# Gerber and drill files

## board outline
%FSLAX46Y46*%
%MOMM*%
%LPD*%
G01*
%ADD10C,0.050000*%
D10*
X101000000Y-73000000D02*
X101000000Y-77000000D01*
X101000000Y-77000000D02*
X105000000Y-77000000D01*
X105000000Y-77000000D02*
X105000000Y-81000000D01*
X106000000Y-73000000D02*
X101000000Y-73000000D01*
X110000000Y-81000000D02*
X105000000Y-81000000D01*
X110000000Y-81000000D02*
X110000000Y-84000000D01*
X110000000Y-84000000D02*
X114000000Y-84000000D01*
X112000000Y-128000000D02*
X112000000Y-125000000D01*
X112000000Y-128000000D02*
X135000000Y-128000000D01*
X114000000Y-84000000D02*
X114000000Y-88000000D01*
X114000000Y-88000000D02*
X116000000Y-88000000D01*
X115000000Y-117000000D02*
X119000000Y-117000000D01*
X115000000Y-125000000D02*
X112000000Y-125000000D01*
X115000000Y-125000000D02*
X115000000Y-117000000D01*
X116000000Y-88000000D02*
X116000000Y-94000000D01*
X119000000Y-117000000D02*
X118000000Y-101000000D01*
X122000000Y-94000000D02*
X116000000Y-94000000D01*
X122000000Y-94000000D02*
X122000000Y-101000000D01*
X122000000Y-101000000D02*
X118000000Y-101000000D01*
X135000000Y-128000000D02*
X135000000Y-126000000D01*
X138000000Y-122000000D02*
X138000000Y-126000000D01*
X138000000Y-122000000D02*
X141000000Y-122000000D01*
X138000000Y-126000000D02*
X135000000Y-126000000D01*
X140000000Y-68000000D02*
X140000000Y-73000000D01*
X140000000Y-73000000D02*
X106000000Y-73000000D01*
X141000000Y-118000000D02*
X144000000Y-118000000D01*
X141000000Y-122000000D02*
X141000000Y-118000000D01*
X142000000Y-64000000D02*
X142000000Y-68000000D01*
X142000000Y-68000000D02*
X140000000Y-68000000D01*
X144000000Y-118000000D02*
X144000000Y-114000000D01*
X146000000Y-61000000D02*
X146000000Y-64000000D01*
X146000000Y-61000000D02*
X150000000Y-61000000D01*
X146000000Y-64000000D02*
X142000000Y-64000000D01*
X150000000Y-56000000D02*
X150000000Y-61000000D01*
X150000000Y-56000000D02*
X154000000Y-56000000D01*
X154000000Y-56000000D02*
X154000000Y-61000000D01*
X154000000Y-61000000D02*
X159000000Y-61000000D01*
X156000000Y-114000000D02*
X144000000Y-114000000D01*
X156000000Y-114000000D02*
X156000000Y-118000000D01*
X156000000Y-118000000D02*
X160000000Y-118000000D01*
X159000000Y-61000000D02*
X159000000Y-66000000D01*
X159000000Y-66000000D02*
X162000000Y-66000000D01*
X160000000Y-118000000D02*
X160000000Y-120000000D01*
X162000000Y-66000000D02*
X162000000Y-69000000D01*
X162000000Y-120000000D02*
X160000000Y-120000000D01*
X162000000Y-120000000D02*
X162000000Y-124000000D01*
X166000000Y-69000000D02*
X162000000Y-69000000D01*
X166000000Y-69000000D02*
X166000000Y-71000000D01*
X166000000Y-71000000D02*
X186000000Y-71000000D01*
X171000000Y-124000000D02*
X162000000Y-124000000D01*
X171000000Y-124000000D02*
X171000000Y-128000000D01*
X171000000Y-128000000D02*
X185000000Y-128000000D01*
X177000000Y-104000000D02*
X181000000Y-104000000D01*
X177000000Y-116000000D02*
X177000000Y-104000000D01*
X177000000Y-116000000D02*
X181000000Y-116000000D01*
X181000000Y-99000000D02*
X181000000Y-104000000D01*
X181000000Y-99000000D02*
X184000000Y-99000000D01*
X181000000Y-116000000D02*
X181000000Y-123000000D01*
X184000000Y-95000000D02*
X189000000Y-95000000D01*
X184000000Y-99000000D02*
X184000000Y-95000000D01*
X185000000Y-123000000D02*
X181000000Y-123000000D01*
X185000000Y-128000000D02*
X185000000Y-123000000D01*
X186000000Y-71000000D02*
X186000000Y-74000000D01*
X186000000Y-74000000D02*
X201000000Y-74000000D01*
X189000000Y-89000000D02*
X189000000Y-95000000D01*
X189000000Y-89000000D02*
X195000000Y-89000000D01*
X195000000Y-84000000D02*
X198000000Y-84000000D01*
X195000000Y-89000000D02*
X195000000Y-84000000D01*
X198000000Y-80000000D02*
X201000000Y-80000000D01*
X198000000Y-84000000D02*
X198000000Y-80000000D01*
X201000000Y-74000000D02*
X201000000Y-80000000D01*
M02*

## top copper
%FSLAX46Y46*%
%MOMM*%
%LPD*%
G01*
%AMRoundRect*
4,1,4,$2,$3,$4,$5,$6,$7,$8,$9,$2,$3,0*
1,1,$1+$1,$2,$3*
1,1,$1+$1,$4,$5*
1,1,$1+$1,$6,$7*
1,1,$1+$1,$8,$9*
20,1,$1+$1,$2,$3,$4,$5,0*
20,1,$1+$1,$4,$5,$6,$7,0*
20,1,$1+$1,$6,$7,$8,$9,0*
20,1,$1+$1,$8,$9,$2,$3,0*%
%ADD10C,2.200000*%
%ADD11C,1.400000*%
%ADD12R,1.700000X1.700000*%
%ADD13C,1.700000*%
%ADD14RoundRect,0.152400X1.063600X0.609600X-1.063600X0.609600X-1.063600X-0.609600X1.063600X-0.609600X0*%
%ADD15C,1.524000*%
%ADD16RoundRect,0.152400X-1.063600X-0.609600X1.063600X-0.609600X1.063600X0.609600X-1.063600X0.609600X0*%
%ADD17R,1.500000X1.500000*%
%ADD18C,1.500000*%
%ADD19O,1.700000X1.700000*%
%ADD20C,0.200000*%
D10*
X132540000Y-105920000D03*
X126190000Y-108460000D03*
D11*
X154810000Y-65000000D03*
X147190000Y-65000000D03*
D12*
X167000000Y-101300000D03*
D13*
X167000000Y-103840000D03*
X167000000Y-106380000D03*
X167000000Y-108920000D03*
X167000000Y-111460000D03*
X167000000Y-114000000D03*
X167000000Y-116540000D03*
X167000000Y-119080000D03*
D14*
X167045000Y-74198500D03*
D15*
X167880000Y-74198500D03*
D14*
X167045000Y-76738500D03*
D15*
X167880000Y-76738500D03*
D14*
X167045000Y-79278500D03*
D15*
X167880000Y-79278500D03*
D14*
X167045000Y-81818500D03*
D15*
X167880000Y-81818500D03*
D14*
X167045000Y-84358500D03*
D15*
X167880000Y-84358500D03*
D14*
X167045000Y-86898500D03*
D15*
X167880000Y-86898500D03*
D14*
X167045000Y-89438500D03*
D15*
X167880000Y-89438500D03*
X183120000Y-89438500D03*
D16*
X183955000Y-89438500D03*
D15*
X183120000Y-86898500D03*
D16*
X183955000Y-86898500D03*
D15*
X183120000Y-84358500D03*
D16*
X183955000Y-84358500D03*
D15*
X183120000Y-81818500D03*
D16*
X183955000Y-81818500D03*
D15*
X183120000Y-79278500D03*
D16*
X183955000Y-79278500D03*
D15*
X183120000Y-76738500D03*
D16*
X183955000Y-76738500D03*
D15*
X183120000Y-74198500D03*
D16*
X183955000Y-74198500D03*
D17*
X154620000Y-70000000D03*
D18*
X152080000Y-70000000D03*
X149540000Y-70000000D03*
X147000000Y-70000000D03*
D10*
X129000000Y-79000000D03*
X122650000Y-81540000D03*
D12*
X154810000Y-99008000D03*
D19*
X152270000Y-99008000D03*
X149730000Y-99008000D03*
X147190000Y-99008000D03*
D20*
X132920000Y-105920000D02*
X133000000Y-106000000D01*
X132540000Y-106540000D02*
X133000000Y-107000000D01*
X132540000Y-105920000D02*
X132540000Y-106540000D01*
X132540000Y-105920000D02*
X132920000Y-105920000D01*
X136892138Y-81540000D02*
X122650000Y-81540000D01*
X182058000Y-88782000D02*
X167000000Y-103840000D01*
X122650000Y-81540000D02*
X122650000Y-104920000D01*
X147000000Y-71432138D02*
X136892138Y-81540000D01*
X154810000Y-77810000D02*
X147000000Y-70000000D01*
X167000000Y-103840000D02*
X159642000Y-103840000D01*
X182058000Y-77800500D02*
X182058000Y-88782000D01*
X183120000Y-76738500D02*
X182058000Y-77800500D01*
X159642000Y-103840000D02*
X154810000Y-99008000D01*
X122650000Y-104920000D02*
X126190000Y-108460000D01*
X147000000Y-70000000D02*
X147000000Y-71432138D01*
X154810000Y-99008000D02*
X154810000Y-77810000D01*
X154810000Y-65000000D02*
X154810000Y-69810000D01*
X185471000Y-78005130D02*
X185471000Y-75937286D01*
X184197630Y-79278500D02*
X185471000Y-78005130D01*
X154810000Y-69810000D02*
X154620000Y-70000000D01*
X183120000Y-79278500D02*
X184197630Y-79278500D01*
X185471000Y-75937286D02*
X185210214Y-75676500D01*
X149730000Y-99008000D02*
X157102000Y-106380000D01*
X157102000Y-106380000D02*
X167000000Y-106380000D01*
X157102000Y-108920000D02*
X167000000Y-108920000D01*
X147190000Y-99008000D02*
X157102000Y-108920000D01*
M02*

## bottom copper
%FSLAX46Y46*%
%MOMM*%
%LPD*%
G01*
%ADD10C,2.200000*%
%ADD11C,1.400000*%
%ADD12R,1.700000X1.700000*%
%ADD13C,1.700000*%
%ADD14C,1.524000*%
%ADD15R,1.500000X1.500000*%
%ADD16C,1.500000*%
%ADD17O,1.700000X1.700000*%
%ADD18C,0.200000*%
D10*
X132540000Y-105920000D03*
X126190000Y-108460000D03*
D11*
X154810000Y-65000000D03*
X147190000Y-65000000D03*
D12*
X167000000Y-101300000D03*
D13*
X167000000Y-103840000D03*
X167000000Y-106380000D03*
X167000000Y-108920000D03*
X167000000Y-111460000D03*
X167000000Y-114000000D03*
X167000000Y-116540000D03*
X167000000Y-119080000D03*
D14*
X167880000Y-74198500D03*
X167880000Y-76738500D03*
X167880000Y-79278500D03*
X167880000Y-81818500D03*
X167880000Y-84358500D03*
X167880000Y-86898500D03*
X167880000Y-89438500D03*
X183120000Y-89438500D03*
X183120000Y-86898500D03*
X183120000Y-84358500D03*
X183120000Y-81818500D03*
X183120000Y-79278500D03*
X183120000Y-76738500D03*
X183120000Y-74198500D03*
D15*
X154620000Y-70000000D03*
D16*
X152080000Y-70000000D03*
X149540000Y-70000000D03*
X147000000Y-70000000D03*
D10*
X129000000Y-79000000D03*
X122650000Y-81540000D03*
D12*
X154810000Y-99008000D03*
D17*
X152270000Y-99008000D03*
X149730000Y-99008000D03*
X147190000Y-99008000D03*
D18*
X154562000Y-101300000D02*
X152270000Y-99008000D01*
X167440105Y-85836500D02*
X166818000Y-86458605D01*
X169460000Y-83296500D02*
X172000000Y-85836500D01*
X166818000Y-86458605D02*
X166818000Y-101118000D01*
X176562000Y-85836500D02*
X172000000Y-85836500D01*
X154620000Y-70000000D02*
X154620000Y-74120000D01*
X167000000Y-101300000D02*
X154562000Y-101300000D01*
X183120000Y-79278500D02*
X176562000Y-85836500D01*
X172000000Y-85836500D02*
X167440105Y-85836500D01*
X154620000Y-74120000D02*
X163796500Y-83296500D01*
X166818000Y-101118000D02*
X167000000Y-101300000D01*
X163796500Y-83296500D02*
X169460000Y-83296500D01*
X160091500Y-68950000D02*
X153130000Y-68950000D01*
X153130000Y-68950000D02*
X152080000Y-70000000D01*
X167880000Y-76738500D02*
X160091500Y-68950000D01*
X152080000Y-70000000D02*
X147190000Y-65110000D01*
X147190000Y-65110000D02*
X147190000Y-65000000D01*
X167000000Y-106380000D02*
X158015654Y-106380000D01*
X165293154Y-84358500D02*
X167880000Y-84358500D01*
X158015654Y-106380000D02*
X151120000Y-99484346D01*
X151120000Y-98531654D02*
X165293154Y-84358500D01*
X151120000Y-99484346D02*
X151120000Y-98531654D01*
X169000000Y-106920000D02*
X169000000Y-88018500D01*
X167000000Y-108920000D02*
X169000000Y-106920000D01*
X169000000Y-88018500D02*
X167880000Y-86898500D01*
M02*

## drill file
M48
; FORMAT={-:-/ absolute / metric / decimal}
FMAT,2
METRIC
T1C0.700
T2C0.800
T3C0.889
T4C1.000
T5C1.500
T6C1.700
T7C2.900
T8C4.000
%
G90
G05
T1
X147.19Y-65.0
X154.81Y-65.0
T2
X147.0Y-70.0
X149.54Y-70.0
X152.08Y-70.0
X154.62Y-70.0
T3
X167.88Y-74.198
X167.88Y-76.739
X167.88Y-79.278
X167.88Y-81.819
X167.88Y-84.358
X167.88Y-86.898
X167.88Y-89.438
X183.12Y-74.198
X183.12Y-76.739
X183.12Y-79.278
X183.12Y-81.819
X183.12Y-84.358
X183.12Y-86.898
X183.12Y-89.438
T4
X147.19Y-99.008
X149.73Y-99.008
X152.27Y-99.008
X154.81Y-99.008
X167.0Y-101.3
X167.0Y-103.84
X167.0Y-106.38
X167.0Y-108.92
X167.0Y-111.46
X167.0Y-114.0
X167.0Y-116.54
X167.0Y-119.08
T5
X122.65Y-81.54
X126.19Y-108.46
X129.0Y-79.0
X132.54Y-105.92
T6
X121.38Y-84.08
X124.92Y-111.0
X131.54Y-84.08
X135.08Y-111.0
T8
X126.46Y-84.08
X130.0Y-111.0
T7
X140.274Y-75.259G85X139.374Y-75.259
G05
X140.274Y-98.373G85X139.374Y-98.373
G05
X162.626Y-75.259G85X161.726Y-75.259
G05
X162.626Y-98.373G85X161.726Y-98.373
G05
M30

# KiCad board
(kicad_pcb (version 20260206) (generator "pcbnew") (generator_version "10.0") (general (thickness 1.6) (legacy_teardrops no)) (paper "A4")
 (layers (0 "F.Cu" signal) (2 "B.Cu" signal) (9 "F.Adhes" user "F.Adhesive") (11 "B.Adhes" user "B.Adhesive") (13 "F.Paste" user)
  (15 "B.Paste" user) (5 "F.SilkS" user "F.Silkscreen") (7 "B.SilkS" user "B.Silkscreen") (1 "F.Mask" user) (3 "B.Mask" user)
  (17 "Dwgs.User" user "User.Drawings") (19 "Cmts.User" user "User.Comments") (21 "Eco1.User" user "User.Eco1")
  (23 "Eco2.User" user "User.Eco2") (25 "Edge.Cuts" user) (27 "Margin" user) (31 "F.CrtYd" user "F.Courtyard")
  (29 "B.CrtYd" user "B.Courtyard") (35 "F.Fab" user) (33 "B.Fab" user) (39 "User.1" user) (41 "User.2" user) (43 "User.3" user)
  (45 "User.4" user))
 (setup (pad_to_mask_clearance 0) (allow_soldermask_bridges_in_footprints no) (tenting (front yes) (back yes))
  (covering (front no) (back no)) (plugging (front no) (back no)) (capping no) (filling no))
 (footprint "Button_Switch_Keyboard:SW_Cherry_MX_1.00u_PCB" (layer "F.Cu") (at 132.54 105.92)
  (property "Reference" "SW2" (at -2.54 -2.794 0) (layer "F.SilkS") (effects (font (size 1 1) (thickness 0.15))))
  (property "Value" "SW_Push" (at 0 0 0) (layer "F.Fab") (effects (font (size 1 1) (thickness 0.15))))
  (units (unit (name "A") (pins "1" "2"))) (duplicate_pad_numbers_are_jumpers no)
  (pad "" np_thru_hole circle (at -7.62 5.08) (size 1.7 1.7) (drill 1.7) (layers "*.Cu" "*.Mask"))
  (pad "" np_thru_hole circle (at -2.54 5.08) (size 4 4) (drill 4) (layers "*.Cu" "*.Mask"))
  (pad "" np_thru_hole circle (at 2.54 5.08) (size 1.7 1.7) (drill 1.7) (layers "*.Cu" "*.Mask"))
  (pad "1" thru_hole circle (at 0 0) (size 2.2 2.2) (drill 1.5) (layers "*.Cu" "*.Mask") (remove_unused_layers no) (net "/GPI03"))
  (pad "2" thru_hole circle (at -6.35 2.54) (size 2.2 2.2) (drill 1.5) (layers "*.Cu" "*.Mask") (remove_unused_layers no) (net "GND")))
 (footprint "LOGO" (layer "F.Cu") (at 160 112)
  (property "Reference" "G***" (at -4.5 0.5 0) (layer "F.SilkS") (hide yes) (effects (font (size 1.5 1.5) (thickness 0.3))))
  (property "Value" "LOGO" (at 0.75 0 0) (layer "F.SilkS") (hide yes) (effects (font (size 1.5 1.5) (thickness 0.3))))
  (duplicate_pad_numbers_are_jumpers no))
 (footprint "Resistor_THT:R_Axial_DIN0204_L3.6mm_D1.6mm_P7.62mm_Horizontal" (layer "F.Cu") (at 154.81 65 180)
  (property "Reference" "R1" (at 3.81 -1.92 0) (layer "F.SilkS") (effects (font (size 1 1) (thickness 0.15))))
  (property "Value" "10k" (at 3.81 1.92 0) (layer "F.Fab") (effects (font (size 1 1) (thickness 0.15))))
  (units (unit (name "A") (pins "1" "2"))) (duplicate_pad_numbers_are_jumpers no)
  (pad "1" thru_hole circle (at 0 0 180) (size 1.4 1.4) (drill 0.7) (layers "*.Cu" "*.Mask") (remove_unused_layers no) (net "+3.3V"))
  (pad "2" thru_hole circle (at 7.62 0 180) (size 1.4 1.4) (drill 0.7) (layers "*.Cu" "*.Mask") (remove_unused_layers no)
   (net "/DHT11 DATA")))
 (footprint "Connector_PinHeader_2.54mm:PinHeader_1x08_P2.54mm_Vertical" (layer "F.Cu") (at 167 101.3)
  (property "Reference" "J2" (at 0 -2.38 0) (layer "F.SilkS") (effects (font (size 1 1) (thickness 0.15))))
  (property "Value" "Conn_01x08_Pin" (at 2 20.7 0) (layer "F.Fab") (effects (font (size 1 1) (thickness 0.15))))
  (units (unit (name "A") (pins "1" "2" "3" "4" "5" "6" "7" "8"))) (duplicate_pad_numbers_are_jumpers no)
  (pad "1" thru_hole rect (at 0 0) (size 1.7 1.7) (drill 1) (layers "*.Cu" "*.Mask") (remove_unused_layers no) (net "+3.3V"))
  (pad "2" thru_hole circle (at 0 2.54) (size 1.7 1.7) (drill 1) (layers "*.Cu" "*.Mask") (remove_unused_layers no) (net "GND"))
  (pad "3" thru_hole circle (at 0 5.08) (size 1.7 1.7) (drill 1) (layers "*.Cu" "*.Mask") (remove_unused_layers no) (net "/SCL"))
  (pad "4" thru_hole circle (at 0 7.62) (size 1.7 1.7) (drill 1) (layers "*.Cu" "*.Mask") (remove_unused_layers no) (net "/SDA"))
  (pad "5" thru_hole circle (at 0 10.16) (size 1.7 1.7) (drill 1) (layers "*.Cu" "*.Mask") (remove_unused_layers no)
   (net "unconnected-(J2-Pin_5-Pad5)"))
  (pad "6" thru_hole circle (at 0 12.7) (size 1.7 1.7) (drill 1) (layers "*.Cu" "*.Mask") (remove_unused_layers no)
   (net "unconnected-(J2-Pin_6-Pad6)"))
  (pad "7" thru_hole circle (at 0 15.24) (size 1.7 1.7) (drill 1) (layers "*.Cu" "*.Mask") (remove_unused_layers no)
   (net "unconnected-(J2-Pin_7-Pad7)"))
  (pad "8" thru_hole circle (at 0 17.78) (size 1.7 1.7) (drill 1) (layers "*.Cu" "*.Mask") (remove_unused_layers no)
   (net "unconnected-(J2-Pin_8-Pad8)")))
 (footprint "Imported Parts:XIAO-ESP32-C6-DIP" (layer "F.Cu") (at 175.5 81.8185 90)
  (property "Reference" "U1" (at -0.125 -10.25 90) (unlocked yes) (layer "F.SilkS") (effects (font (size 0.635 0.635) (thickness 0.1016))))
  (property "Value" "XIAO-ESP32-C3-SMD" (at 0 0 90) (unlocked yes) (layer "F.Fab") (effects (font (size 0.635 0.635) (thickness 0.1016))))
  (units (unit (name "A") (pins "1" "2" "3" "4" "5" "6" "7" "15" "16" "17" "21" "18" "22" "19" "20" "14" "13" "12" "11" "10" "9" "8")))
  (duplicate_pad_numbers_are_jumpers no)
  (pad "1" smd roundrect (at 7.62 -8.455 180) (size 2.432 1.524) (layers "F.Cu" "F.Mask") (roundrect_rratio 0.1)
   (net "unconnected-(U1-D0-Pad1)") (thermal_bridge_angle 45))
  (pad "1" thru_hole circle (at 7.62 -7.62 180) (size 1.524 1.524) (drill 0.889) (layers "*.Cu" "*.Mask") (remove_unused_layers no)
   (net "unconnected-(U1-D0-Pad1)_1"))
  (pad "2" smd roundrect (at 5.08 -8.455 180) (size 2.432 1.524) (layers "F.Cu" "F.Mask") (roundrect_rratio 0.1) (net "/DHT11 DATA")
   (thermal_bridge_angle 45))
  (pad "2" thru_hole circle (at 5.08 -7.62 180) (size 1.524 1.524) (drill 0.889) (layers "*.Cu" "*.Mask") (remove_unused_layers no)
   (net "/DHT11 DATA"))
  (pad "3" smd roundrect (at 2.54 -8.455 180) (size 2.432 1.524) (layers "F.Cu" "F.Mask") (roundrect_rratio 0.1) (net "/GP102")
   (thermal_bridge_angle 45))
  (pad "3" thru_hole circle (at 2.54 -7.62 180) (size 1.524 1.524) (drill 0.889) (layers "*.Cu" "*.Mask") (remove_unused_layers no)
   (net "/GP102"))
  (pad "4" smd roundrect (at 0 -8.455 180) (size 2.432 1.524) (layers "F.Cu" "F.Mask") (roundrect_rratio 0.1) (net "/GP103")
   (thermal_bridge_angle 45))
  (pad "4" thru_hole circle (at 0 -7.62 180) (size 1.524 1.524) (drill 0.889) (layers "*.Cu" "*.Mask") (remove_unused_layers no)
   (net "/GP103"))
  (pad "5" smd roundrect (at -2.54 -8.455 180) (size 2.432 1.524) (layers "F.Cu" "F.Mask") (roundrect_rratio 0.1) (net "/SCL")
   (thermal_bridge_angle 45))
  (pad "5" thru_hole circle (at -2.54 -7.62 180) (size 1.524 1.524) (drill 0.889) (layers "*.Cu" "*.Mask") (remove_unused_layers no)
   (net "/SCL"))
  (pad "6" smd roundrect (at -5.08 -8.455 180) (size 2.432 1.524) (layers "F.Cu" "F.Mask") (roundrect_rratio 0.1) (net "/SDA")
   (thermal_bridge_angle 45))
  (pad "6" thru_hole circle (at -5.08 -7.62 180) (size 1.524 1.524) (drill 0.889) (layers "*.Cu" "*.Mask") (remove_unused_layers no)
   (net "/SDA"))
  (pad "7" smd roundrect (at -7.62 -8.455 180) (size 2.432 1.524) (layers "F.Cu" "F.Mask") (roundrect_rratio 0.1)
   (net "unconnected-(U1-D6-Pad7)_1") (thermal_bridge_angle 45))
  (pad "7" thru_hole circle (at -7.62 -7.62 180) (size 1.524 1.524) (drill 0.889) (layers "*.Cu" "*.Mask") (remove_unused_layers no)
   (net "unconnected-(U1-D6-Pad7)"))
  (pad "8" thru_hole circle (at -7.62 7.62) (size 1.524 1.524) (drill 0.889) (layers "*.Cu" "*.Mask") (remove_unused_layers no)
   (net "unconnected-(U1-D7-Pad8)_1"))
  (pad "8" smd roundrect (at -7.62 8.455) (size 2.432 1.524) (layers "F.Cu" "F.Mask") (roundrect_rratio 0.1)
   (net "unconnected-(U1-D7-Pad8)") (thermal_bridge_angle 45))
  (pad "9" thru_hole circle (at -5.08 7.62) (size 1.524 1.524) (drill 0.889) (layers "*.Cu" "*.Mask") (remove_unused_layers no)
   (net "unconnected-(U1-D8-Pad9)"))
  (pad "9" smd roundrect (at -5.08 8.455) (size 2.432 1.524) (layers "F.Cu" "F.Mask") (roundrect_rratio 0.1)
   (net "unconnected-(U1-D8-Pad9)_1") (thermal_bridge_angle 45))
  (pad "10" thru_hole circle (at -2.54 7.62) (size 1.524 1.524) (drill 0.889) (layers "*.Cu" "*.Mask") (remove_unused_layers no)
   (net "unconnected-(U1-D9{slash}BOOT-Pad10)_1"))
  (pad "10" smd roundrect (at -2.54 8.455) (size 2.432 1.524) (layers "F.Cu" "F.Mask") (roundrect_rratio 0.1)
   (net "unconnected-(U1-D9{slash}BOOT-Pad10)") (thermal_bridge_angle 45))
  (pad "11" thru_hole circle (at 0 7.62) (size 1.524 1.524) (drill 0.889) (layers "*.Cu" "*.Mask") (remove_unused_layers no)
   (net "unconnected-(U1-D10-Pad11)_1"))
  (pad "11" smd roundrect (at 0 8.455) (size 2.432 1.524) (layers "F.Cu" "F.Mask") (roundrect_rratio 0.1) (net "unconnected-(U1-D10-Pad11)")
   (thermal_bridge_angle 45))
  (pad "12" thru_hole circle (at 2.54 7.62) (size 1.524 1.524) (drill 0.889) (layers "*.Cu" "*.Mask") (remove_unused_layers no)
   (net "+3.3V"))
  (pad "12" smd roundrect (at 2.54 8.455) (size 2.432 1.524) (layers "F.Cu" "F.Mask") (roundrect_rratio 0.1) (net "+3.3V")
   (thermal_bridge_angle 45))
  (pad "13" thru_hole circle (at 5.08 7.62) (size 1.524 1.524) (drill 0.889) (layers "*.Cu" "*.Mask") (remove_unused_layers no) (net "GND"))
  (pad "13" smd roundrect (at 5.08 8.455) (size 2.432 1.524) (layers "F.Cu" "F.Mask") (roundrect_rratio 0.1) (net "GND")
   (thermal_bridge_angle 45))
  (pad "14" thru_hole circle (at 7.62 7.62) (size 1.524 1.524) (drill 0.889) (layers "*.Cu" "*.Mask") (remove_unused_layers no) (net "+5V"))
  (pad "14" smd roundrect (at 7.62 8.455) (size 2.432 1.524) (layers "F.Cu" "F.Mask") (roundrect_rratio 0.1) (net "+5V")
   (thermal_bridge_angle 45)))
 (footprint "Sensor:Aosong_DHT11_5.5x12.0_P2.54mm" (layer "F.Cu") (at 154.62 70 -90)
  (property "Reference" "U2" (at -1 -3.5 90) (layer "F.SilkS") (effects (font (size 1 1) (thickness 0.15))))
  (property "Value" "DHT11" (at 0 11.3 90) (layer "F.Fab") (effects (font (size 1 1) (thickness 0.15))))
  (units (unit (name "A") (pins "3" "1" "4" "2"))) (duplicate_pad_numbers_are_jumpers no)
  (pad "1" thru_hole rect (at 0 0 270) (size 1.5 1.5) (drill 0.8) (layers "*.Cu" "*.Mask") (remove_unused_layers no) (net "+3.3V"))
  (pad "2" thru_hole circle (at 0 2.54 270) (size 1.5 1.5) (drill 0.8) (layers "*.Cu" "*.Mask") (remove_unused_layers no)
   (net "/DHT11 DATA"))
  (pad "3" thru_hole circle (at 0 5.08 270) (size 1.5 1.5) (drill 0.8) (layers "*.Cu" "*.Mask") (remove_unused_layers no)
   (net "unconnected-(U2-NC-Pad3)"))
  (pad "4" thru_hole circle (at 0 7.62 270) (size 1.5 1.5) (drill 0.8) (layers "*.Cu" "*.Mask") (remove_unused_layers no) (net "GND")))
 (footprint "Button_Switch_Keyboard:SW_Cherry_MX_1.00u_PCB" (layer "F.Cu") (at 129 79)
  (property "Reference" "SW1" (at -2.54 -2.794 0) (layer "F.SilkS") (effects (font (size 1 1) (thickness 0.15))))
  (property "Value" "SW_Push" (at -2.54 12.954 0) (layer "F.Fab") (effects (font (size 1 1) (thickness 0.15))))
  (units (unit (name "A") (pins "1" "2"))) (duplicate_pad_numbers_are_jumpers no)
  (pad "" np_thru_hole circle (at -7.62 5.08) (size 1.7 1.7) (drill 1.7) (layers "*.Cu" "*.Mask"))
  (pad "" np_thru_hole circle (at -2.54 5.08) (size 4 4) (drill 4) (layers "*.Cu" "*.Mask"))
  (pad "" np_thru_hole circle (at 2.54 5.08) (size 1.7 1.7) (drill 1.7) (layers "*.Cu" "*.Mask"))
  (pad "1" thru_hole circle (at 0 0) (size 2.2 2.2) (drill 1.5) (layers "*.Cu" "*.Mask") (remove_unused_layers no) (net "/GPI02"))
  (pad "2" thru_hole circle (at -6.35 2.54) (size 2.2 2.2) (drill 1.5) (layers "*.Cu" "*.Mask") (remove_unused_layers no) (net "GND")))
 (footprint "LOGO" (layer "F.Cu") (at 191.5 80.5)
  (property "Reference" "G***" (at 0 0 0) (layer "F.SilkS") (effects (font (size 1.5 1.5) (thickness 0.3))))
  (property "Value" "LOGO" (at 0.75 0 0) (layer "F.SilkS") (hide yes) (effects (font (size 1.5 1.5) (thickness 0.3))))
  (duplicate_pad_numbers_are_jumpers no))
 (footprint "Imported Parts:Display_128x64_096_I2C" (layer "F.Cu") (at 151 99.008 180)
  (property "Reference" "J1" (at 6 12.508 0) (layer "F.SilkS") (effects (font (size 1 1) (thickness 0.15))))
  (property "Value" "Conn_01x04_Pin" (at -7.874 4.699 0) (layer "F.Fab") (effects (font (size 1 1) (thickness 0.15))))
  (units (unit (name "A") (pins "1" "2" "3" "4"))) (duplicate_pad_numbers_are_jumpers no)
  (pad "" np_thru_hole oval (at -11.176 0.635 180) (size 3.8 2.9) (drill oval 3.8 2.9) (layers "*.Cu" "*.Mask"))
  (pad "" np_thru_hole oval (at -11.176 23.749 180) (size 3.8 2.9) (drill oval 3.8 2.9) (layers "*.Cu" "*.Mask"))
  (pad "" np_thru_hole oval (at 11.176 0.635 180) (size 3.8 2.9) (drill oval 3.8 2.9) (layers "*.Cu" "*.Mask"))
  (pad "" np_thru_hole oval (at 11.176 23.749 180) (size 3.8 2.9) (drill oval 3.8 2.9) (layers "*.Cu" "*.Mask"))
  (pad "1" thru_hole rect (at -3.81 0 270) (size 1.7 1.7) (drill 1) (layers "*.Cu" "*.Mask") (remove_unused_layers no) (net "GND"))
  (pad "2" thru_hole oval (at -1.27 0 270) (size 1.7 1.7) (drill 1) (layers "*.Cu" "*.Mask") (remove_unused_layers no) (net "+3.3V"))
  (pad "3" thru_hole oval (at 1.27 0 270) (size 1.7 1.7) (drill 1) (layers "*.Cu" "*.Mask") (remove_unused_layers no) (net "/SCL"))
  (pad "4" thru_hole oval (at 3.81 0 270) (size 1.7 1.7) (drill 1) (layers "*.Cu" "*.Mask") (remove_unused_layers no) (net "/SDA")))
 (gr_line (start 101 73) (end 101 77) (stroke (width 0.05) (type default)) (layer "Edge.Cuts"))
 (gr_line (start 101 77) (end 105 77) (stroke (width 0.05) (type default)) (layer "Edge.Cuts"))
 (gr_line (start 105 77) (end 105 81) (stroke (width 0.05) (type default)) (layer "Edge.Cuts"))
 (gr_line (start 106 73) (end 101 73) (stroke (width 0.05) (type default)) (layer "Edge.Cuts"))
 (gr_line (start 110 81) (end 105 81) (stroke (width 0.05) (type default)) (layer "Edge.Cuts"))
 (gr_line (start 110 81) (end 110 84) (stroke (width 0.05) (type default)) (layer "Edge.Cuts"))
 (gr_line (start 110 84) (end 114 84) (stroke (width 0.05) (type default)) (layer "Edge.Cuts"))
 (gr_line (start 112 128) (end 112 125) (stroke (width 0.05) (type default)) (layer "Edge.Cuts"))
 (gr_line (start 112 128) (end 135 128) (stroke (width 0.05) (type default)) (layer "Edge.Cuts"))
 (gr_line (start 114 84) (end 114 88) (stroke (width 0.05) (type default)) (layer "Edge.Cuts"))
 (gr_line (start 114 88) (end 116 88) (stroke (width 0.05) (type default)) (layer "Edge.Cuts"))
 (gr_line (start 115 117) (end 119 117) (stroke (width 0.05) (type default)) (layer "Edge.Cuts"))
 (gr_line (start 115 125) (end 112 125) (stroke (width 0.05) (type default)) (layer "Edge.Cuts"))
 (gr_line (start 115 125) (end 115 117) (stroke (width 0.05) (type default)) (layer "Edge.Cuts"))
 (gr_line (start 116 88) (end 116 94) (stroke (width 0.05) (type default)) (layer "Edge.Cuts"))
 (gr_line (start 119 117) (end 118 101) (stroke (width 0.05) (type default)) (layer "Edge.Cuts"))
 (gr_line (start 122 94) (end 116 94) (stroke (width 0.05) (type default)) (layer "Edge.Cuts"))
 (gr_line (start 122 94) (end 122 101) (stroke (width 0.05) (type default)) (layer "Edge.Cuts"))
 (gr_line (start 122 101) (end 118 101) (stroke (width 0.05) (type default)) (layer "Edge.Cuts"))
 (gr_line (start 135 128) (end 135 126) (stroke (width 0.05) (type default)) (layer "Edge.Cuts"))
 (gr_line (start 138 122) (end 138 126) (stroke (width 0.05) (type default)) (layer "Edge.Cuts"))
 (gr_line (start 138 122) (end 141 122) (stroke (width 0.05) (type default)) (layer "Edge.Cuts"))
 (gr_line (start 138 126) (end 135 126) (stroke (width 0.05) (type default)) (layer "Edge.Cuts"))
 (gr_line (start 140 68) (end 140 73) (stroke (width 0.05) (type default)) (layer "Edge.Cuts"))
 (gr_line (start 140 73) (end 106 73) (stroke (width 0.05) (type default)) (layer "Edge.Cuts"))
 (gr_line (start 141 118) (end 144 118) (stroke (width 0.05) (type default)) (layer "Edge.Cuts"))
 (gr_line (start 141 122) (end 141 118) (stroke (width 0.05) (type default)) (layer "Edge.Cuts"))
 (gr_line (start 142 64) (end 142 68) (stroke (width 0.05) (type default)) (layer "Edge.Cuts"))
 (gr_line (start 142 68) (end 140 68) (stroke (width 0.05) (type default)) (layer "Edge.Cuts"))
 (gr_line (start 144 118) (end 144 114) (stroke (width 0.05) (type default)) (layer "Edge.Cuts"))
 (gr_line (start 146 61) (end 146 64) (stroke (width 0.05) (type default)) (layer "Edge.Cuts"))
 (gr_line (start 146 61) (end 150 61) (stroke (width 0.05) (type default)) (layer "Edge.Cuts"))
 (gr_line (start 146 64) (end 142 64) (stroke (width 0.05) (type default)) (layer "Edge.Cuts"))
 (gr_line (start 150 56) (end 150 61) (stroke (width 0.05) (type default)) (layer "Edge.Cuts"))
 (gr_line (start 150 56) (end 154 56) (stroke (width 0.05) (type default)) (layer "Edge.Cuts"))
 (gr_line (start 154 56) (end 154 61) (stroke (width 0.05) (type default)) (layer "Edge.Cuts"))
 (gr_line (start 154 61) (end 159 61) (stroke (width 0.05) (type default)) (layer "Edge.Cuts"))
 (gr_line (start 156 114) (end 144 114) (stroke (width 0.05) (type default)) (layer "Edge.Cuts"))
 (gr_line (start 156 114) (end 156 118) (stroke (width 0.05) (type default)) (layer "Edge.Cuts"))
 (gr_line (start 156 118) (end 160 118) (stroke (width 0.05) (type default)) (layer "Edge.Cuts"))
 (gr_line (start 159 61) (end 159 66) (stroke (width 0.05) (type default)) (layer "Edge.Cuts"))
 (gr_line (start 159 66) (end 162 66) (stroke (width 0.05) (type default)) (layer "Edge.Cuts"))
 (gr_line (start 160 118) (end 160 120) (stroke (width 0.05) (type default)) (layer "Edge.Cuts"))
 (gr_line (start 162 66) (end 162 69) (stroke (width 0.05) (type default)) (layer "Edge.Cuts"))
 (gr_line (start 162 120) (end 160 120) (stroke (width 0.05) (type default)) (layer "Edge.Cuts"))
 (gr_line (start 162 120) (end 162 124) (stroke (width 0.05) (type default)) (layer "Edge.Cuts"))
 (gr_line (start 166 69) (end 162 69) (stroke (width 0.05) (type default)) (layer "Edge.Cuts"))
 (gr_line (start 166 69) (end 166 71) (stroke (width 0.05) (type default)) (layer "Edge.Cuts"))
 (gr_line (start 166 71) (end 186 71) (stroke (width 0.05) (type default)) (layer "Edge.Cuts"))
 (gr_line (start 171 124) (end 162 124) (stroke (width 0.05) (type default)) (layer "Edge.Cuts"))
 (gr_line (start 171 124) (end 171 128) (stroke (width 0.05) (type default)) (layer "Edge.Cuts"))
 (gr_line (start 171 128) (end 185 128) (stroke (width 0.05) (type default)) (layer "Edge.Cuts"))
 (gr_line (start 177 104) (end 181 104) (stroke (width 0.05) (type default)) (layer "Edge.Cuts"))
 (gr_line (start 177 116) (end 177 104) (stroke (width 0.05) (type default)) (layer "Edge.Cuts"))
 (gr_line (start 177 116) (end 181 116) (stroke (width 0.05) (type default)) (layer "Edge.Cuts"))
 (gr_line (start 181 99) (end 181 104) (stroke (width 0.05) (type default)) (layer "Edge.Cuts"))
 (gr_line (start 181 99) (end 184 99) (stroke (width 0.05) (type default)) (layer "Edge.Cuts"))
 (gr_line (start 181 116) (end 181 123) (stroke (width 0.05) (type default)) (layer "Edge.Cuts"))
 (gr_line (start 184 95) (end 189 95) (stroke (width 0.05) (type default)) (layer "Edge.Cuts"))
 (gr_line (start 184 99) (end 184 95) (stroke (width 0.05) (type default)) (layer "Edge.Cuts"))
 (gr_line (start 185 123) (end 181 123) (stroke (width 0.05) (type default)) (layer "Edge.Cuts"))
 (gr_line (start 185 128) (end 185 123) (stroke (width 0.05) (type default)) (layer "Edge.Cuts"))
 (gr_line (start 186 71) (end 186 74) (stroke (width 0.05) (type default)) (layer "Edge.Cuts"))
 (gr_line (start 186 74) (end 201 74) (stroke (width 0.05) (type default)) (layer "Edge.Cuts"))
 (gr_line (start 189 89) (end 189 95) (stroke (width 0.05) (type default)) (layer "Edge.Cuts"))
 (gr_line (start 189 89) (end 195 89) (stroke (width 0.05) (type default)) (layer "Edge.Cuts"))
 (gr_line (start 195 84) (end 198 84) (stroke (width 0.05) (type default)) (layer "Edge.Cuts"))
 (gr_line (start 195 89) (end 195 84) (stroke (width 0.05) (type default)) (layer "Edge.Cuts"))
 (gr_line (start 198 80) (end 201 80) (stroke (width 0.05) (type default)) (layer "Edge.Cuts"))
 (gr_line (start 198 84) (end 198 80) (stroke (width 0.05) (type default)) (layer "Edge.Cuts"))
 (gr_line (start 201 74) (end 201 80) (stroke (width 0.05) (type default)) (layer "Edge.Cuts"))
 (segment (start 132.92 105.92) (end 133 106) (width 0.2) (layer "F.Cu") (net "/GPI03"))
 (segment (start 132.54 106.54) (end 133 107) (width 0.2) (layer "F.Cu") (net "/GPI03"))
 (segment (start 132.54 105.92) (end 132.54 106.54) (width 0.2) (layer "F.Cu") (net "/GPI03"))
 (segment (start 132.54 105.92) (end 132.92 105.92) (width 0.2) (layer "F.Cu") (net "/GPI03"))
 (segment (start 136.892138 81.54) (end 122.65 81.54) (width 0.2) (layer "F.Cu") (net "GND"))
 (segment (start 182.058 88.782) (end 167 103.84) (width 0.2) (layer "F.Cu") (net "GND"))
 (segment (start 122.65 81.54) (end 122.65 104.92) (width 0.2) (layer "F.Cu") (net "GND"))
 (segment (start 147 71.432138) (end 136.892138 81.54) (width 0.2) (layer "F.Cu") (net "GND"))
 (segment (start 154.81 77.81) (end 147 70) (width 0.2) (layer "F.Cu") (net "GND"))
 (segment (start 167 103.84) (end 159.642 103.84) (width 0.2) (layer "F.Cu") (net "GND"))
 (segment (start 182.058 77.8005) (end 182.058 88.782) (width 0.2) (layer "F.Cu") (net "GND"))
 (segment (start 183.12 76.7385) (end 182.058 77.8005) (width 0.2) (layer "F.Cu") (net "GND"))
 (segment (start 159.642 103.84) (end 154.81 99.008) (width 0.2) (layer "F.Cu") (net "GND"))
 (segment (start 122.65 104.92) (end 126.19 108.46) (width 0.2) (layer "F.Cu") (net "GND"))
 (segment (start 147 70) (end 147 71.432138) (width 0.2) (layer "F.Cu") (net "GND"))
 (segment (start 154.81 99.008) (end 154.81 77.81) (width 0.2) (layer "F.Cu") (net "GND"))
 (segment (start 154.81 65) (end 154.81 69.81) (width 0.2) (layer "F.Cu") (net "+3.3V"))
 (segment (start 185.471 78.00513) (end 185.471 75.937286) (width 0.2) (layer "F.Cu") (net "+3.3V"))
 (segment (start 184.19763 79.2785) (end 185.471 78.00513) (width 0.2) (layer "F.Cu") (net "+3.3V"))
 (segment (start 154.81 69.81) (end 154.62 70) (width 0.2) (layer "F.Cu") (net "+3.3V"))
 (segment (start 183.12 79.2785) (end 184.19763 79.2785) (width 0.2) (layer "F.Cu") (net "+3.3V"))
 (segment (start 185.471 75.937286) (end 185.210214 75.6765) (width 0.2) (layer "F.Cu") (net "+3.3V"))
 (segment (start 154.562 101.3) (end 152.27 99.008) (width 0.2) (layer "B.Cu") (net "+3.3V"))
 (segment (start 167.440105 85.8365) (end 166.818 86.458605) (width 0.2) (layer "B.Cu") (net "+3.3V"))
 (segment (start 169.46 83.2965) (end 172 85.8365) (width 0.2) (layer "B.Cu") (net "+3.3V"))
 (segment (start 166.818 86.458605) (end 166.818 101.118) (width 0.2) (layer "B.Cu") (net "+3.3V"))
 (segment (start 176.562 85.8365) (end 172 85.8365) (width 0.2) (layer "B.Cu") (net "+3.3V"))
 (segment (start 154.62 70) (end 154.62 74.12) (width 0.2) (layer "B.Cu") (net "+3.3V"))
 (segment (start 167 101.3) (end 154.562 101.3) (width 0.2) (layer "B.Cu") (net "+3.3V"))
 (segment (start 183.12 79.2785) (end 176.562 85.8365) (width 0.2) (layer "B.Cu") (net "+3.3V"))
 (segment (start 172 85.8365) (end 167.440105 85.8365) (width 0.2) (layer "B.Cu") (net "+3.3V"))
 (segment (start 154.62 74.12) (end 163.7965 83.2965) (width 0.2) (layer "B.Cu") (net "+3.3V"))
 (segment (start 166.818 101.118) (end 167 101.3) (width 0.2) (layer "B.Cu") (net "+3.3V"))
 (segment (start 163.7965 83.2965) (end 169.46 83.2965) (width 0.2) (layer "B.Cu") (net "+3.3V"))
 (segment (start 160.0915 68.95) (end 153.13 68.95) (width 0.2) (layer "B.Cu") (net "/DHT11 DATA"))
 (segment (start 153.13 68.95) (end 152.08 70) (width 0.2) (layer "B.Cu") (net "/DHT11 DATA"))
 (segment (start 167.88 76.7385) (end 160.0915 68.95) (width 0.2) (layer "B.Cu") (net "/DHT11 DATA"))
 (segment (start 152.08 70) (end 147.19 65.11) (width 0.2) (layer "B.Cu") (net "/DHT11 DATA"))
 (segment (start 147.19 65.11) (end 147.19 65) (width 0.2) (layer "B.Cu") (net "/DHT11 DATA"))
 (segment (start 149.73 99.008) (end 157.102 106.38) (width 0.2) (layer "F.Cu") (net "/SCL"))
 (segment (start 157.102 106.38) (end 167 106.38) (width 0.2) (layer "F.Cu") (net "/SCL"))
 (segment (start 167 106.38) (end 158.015654 106.38) (width 0.2) (layer "B.Cu") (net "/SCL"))
 (segment (start 165.293154 84.3585) (end 167.88 84.3585) (width 0.2) (layer "B.Cu") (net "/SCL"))
 (segment (start 158.015654 106.38) (end 151.12 99.484346) (width 0.2) (layer "B.Cu") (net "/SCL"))
 (segment (start 151.12 98.531654) (end 165.293154 84.3585) (width 0.2) (layer "B.Cu") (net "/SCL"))
 (segment (start 151.12 99.484346) (end 151.12 98.531654) (width 0.2) (layer "B.Cu") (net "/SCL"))
 (segment (start 157.102 108.92) (end 167 108.92) (width 0.2) (layer "F.Cu") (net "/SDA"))
 (segment (start 147.19 99.008) (end 157.102 108.92) (width 0.2) (layer "F.Cu") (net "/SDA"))
 (segment (start 169 106.92) (end 169 88.0185) (width 0.2) (layer "B.Cu") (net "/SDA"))
 (segment (start 167 108.92) (end 169 106.92) (width 0.2) (layer "B.Cu") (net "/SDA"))
 (segment (start 169 88.0185) (end 167.88 86.8985) (width 0.2) (layer "B.Cu") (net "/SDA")))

